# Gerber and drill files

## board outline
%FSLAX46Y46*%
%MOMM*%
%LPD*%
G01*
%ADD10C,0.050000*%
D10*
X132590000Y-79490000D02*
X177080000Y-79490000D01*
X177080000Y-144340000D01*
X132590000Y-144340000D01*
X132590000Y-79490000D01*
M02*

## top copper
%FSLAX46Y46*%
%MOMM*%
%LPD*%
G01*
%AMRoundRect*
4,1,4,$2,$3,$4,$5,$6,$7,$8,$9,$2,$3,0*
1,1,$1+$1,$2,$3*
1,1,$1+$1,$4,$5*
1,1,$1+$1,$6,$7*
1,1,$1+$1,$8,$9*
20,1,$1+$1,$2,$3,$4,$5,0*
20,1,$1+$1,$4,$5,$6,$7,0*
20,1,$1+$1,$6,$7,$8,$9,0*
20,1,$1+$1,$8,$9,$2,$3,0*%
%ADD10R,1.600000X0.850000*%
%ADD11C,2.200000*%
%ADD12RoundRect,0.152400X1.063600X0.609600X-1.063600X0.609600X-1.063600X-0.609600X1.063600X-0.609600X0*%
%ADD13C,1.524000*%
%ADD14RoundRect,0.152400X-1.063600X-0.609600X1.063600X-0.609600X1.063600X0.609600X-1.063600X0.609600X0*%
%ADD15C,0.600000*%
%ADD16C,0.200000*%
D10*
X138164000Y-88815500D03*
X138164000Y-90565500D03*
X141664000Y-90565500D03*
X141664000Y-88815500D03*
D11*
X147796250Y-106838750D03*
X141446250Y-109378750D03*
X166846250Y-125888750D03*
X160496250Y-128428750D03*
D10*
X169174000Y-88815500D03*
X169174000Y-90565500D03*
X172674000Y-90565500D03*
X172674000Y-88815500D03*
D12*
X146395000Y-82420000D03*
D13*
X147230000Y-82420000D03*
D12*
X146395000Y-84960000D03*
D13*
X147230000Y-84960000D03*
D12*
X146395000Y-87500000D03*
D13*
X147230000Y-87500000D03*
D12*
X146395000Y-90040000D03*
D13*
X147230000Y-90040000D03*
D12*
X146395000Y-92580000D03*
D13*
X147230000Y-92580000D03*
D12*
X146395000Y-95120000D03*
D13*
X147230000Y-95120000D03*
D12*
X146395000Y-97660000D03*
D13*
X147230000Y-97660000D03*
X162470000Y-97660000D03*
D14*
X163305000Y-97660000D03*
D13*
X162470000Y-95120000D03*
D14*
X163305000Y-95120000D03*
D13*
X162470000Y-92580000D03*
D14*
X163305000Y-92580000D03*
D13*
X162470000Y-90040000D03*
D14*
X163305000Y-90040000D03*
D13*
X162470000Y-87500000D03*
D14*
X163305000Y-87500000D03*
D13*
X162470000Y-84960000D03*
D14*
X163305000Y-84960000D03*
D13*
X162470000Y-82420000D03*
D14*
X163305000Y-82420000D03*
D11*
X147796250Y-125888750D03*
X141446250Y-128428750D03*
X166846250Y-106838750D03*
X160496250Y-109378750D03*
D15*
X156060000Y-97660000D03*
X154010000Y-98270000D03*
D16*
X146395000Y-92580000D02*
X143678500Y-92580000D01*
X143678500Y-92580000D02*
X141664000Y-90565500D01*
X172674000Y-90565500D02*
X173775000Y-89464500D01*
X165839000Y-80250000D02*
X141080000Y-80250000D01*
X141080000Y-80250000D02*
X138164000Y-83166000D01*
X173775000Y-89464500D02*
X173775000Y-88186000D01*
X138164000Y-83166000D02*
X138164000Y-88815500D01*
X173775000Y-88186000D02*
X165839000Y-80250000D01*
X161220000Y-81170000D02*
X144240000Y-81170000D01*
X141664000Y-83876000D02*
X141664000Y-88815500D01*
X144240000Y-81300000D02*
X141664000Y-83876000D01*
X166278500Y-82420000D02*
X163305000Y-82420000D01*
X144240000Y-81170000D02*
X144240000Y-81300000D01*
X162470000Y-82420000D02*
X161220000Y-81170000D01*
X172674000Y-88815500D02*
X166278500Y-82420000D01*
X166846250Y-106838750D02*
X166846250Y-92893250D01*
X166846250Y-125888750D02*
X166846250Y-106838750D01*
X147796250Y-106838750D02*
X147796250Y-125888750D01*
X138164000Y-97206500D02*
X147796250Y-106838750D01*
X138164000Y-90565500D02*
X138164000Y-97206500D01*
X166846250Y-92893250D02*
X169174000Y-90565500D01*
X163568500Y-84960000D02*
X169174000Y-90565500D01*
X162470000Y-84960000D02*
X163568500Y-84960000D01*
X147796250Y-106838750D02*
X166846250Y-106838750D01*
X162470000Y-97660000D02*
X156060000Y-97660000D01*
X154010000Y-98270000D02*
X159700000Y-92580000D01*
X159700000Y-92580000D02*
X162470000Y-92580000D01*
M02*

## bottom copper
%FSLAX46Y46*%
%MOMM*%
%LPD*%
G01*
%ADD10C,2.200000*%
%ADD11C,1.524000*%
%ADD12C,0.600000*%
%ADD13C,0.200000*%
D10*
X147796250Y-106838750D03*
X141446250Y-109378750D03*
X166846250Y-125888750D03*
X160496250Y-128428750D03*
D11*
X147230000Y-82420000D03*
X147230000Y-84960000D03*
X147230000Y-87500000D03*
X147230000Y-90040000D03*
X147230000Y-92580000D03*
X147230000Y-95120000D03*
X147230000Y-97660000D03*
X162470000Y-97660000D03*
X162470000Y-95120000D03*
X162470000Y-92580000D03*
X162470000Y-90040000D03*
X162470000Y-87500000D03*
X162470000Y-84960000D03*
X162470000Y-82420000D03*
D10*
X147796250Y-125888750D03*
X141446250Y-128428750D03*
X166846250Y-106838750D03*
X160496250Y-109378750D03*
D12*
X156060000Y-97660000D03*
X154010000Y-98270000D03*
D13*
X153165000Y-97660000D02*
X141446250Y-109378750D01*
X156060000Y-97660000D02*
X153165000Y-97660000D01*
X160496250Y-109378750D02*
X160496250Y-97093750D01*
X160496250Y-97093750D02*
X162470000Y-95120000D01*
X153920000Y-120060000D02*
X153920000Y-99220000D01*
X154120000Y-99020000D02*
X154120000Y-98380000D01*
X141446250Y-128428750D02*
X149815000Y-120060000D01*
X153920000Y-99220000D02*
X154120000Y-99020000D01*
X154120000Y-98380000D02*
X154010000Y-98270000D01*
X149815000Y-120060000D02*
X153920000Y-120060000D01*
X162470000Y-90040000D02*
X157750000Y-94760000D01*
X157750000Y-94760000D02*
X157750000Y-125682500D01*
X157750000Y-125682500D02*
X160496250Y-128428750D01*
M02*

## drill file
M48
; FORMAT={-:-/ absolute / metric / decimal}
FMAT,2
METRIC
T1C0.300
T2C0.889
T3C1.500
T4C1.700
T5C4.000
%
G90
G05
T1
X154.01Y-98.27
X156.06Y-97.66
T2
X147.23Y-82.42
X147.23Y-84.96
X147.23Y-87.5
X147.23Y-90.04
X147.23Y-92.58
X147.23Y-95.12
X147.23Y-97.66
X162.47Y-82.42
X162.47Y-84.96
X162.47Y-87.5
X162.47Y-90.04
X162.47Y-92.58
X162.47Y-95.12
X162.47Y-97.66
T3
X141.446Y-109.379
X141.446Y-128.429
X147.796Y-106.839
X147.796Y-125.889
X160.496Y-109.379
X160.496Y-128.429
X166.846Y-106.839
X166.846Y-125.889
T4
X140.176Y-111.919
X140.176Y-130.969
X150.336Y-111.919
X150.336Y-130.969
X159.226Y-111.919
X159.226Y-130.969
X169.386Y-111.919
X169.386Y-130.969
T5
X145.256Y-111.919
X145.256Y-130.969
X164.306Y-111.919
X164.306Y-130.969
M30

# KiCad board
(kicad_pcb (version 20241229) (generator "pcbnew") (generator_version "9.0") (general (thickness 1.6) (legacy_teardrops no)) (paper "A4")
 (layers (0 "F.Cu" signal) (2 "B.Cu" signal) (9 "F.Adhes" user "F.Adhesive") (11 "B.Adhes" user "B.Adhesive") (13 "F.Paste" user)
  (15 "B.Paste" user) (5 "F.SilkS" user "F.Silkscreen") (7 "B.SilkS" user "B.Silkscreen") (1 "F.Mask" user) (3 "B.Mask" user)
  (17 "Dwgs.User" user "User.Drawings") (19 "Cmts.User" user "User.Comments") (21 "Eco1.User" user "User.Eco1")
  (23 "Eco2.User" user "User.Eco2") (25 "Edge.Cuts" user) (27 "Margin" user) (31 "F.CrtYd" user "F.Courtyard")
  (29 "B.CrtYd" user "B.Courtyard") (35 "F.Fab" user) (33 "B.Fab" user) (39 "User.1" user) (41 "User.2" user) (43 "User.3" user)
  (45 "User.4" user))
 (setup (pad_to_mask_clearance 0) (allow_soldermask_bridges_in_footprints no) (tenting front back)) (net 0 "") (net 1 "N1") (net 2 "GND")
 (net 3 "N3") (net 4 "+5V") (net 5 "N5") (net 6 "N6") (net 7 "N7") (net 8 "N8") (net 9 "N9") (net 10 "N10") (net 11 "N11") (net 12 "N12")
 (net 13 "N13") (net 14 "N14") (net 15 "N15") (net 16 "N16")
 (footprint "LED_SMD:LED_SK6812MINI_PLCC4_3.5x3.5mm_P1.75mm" (layer "F.Cu") (at 139.914 89.6905)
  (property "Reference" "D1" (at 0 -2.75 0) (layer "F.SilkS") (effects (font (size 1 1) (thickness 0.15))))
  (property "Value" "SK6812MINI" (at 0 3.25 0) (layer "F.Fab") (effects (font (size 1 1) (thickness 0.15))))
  (pad "1" smd rect (at -1.75 -0.875) (size 1.6 0.85) (layers "F.Cu" "F.Mask" "F.Paste") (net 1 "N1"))
  (pad "2" smd rect (at -1.75 0.875) (size 1.6 0.85) (layers "F.Cu" "F.Mask" "F.Paste") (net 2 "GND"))
  (pad "3" smd rect (at 1.75 0.875) (size 1.6 0.85) (layers "F.Cu" "F.Mask" "F.Paste") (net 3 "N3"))
  (pad "4" smd rect (at 1.75 -0.875) (size 1.6 0.85) (layers "F.Cu" "F.Mask" "F.Paste") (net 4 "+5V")))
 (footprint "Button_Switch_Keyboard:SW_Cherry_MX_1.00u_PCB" (layer "F.Cu") (at 147.79625 106.83875)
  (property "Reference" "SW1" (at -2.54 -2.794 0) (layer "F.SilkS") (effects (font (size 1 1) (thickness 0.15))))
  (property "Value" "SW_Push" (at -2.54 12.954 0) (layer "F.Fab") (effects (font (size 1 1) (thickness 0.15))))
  (pad "" np_thru_hole circle (at -7.62 5.08) (size 1.7 1.7) (drill 1.7) (layers "*.Cu" "*.Mask"))
  (pad "" np_thru_hole circle (at -2.54 5.08) (size 4 4) (drill 4) (layers "*.Cu" "*.Mask"))
  (pad "" np_thru_hole circle (at 2.54 5.08) (size 1.7 1.7) (drill 1.7) (layers "*.Cu" "*.Mask"))
  (pad "1" thru_hole circle (at 0 0) (size 2.2 2.2) (drill 1.5) (layers "*.Cu" "*.Mask") (remove_unused_layers no) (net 2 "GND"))
  (pad "2" thru_hole circle (at -6.35 2.54) (size 2.2 2.2) (drill 1.5) (layers "*.Cu" "*.Mask") (remove_unused_layers no) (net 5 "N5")))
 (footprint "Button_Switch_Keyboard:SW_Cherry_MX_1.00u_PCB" (layer "F.Cu") (at 166.84625 125.88875)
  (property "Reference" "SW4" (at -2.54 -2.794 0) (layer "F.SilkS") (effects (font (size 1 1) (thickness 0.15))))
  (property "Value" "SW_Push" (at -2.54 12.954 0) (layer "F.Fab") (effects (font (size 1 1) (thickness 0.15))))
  (pad "" np_thru_hole circle (at -7.62 5.08) (size 1.7 1.7) (drill 1.7) (layers "*.Cu" "*.Mask"))
  (pad "" np_thru_hole circle (at -2.54 5.08) (size 4 4) (drill 4) (layers "*.Cu" "*.Mask"))
  (pad "" np_thru_hole circle (at 2.54 5.08) (size 1.7 1.7) (drill 1.7) (layers "*.Cu" "*.Mask"))
  (pad "1" thru_hole circle (at 0 0) (size 2.2 2.2) (drill 1.5) (layers "*.Cu" "*.Mask") (remove_unused_layers no) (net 2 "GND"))
  (pad "2" thru_hole circle (at -6.35 2.54) (size 2.2 2.2) (drill 1.5) (layers "*.Cu" "*.Mask") (remove_unused_layers no) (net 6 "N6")))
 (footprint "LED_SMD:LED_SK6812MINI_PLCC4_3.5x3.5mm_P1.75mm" (layer "F.Cu") (at 170.924 89.6905)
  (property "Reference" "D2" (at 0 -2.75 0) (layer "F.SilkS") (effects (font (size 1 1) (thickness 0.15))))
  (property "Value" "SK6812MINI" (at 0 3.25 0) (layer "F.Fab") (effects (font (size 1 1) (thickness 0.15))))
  (pad "1" smd rect (at -1.75 -0.875) (size 1.6 0.85) (layers "F.Cu" "F.Mask" "F.Paste") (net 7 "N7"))
  (pad "2" smd rect (at -1.75 0.875) (size 1.6 0.85) (layers "F.Cu" "F.Mask" "F.Paste") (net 2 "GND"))
  (pad "3" smd rect (at 1.75 0.875) (size 1.6 0.85) (layers "F.Cu" "F.Mask" "F.Paste") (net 1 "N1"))
  (pad "4" smd rect (at 1.75 -0.875) (size 1.6 0.85) (layers "F.Cu" "F.Mask" "F.Paste") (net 4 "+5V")))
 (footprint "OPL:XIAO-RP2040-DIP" (layer "F.Cu") (at 154.85 90.04)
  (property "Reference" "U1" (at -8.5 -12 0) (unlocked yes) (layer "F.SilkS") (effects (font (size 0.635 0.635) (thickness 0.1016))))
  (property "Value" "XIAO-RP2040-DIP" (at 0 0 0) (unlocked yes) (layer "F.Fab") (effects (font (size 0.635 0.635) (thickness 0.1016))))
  (pad "1" smd roundrect (at -8.455 -7.62 180) (size 2.432 1.524) (layers "F.Cu" "F.Mask") (roundrect_rratio 0.1) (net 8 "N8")
   (thermal_bridge_angle 45))
  (pad "1" thru_hole circle (at -7.62 -7.62 180) (size 1.524 1.524) (drill 0.889) (layers "*.Cu" "*.Mask") (remove_unused_layers no)
   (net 8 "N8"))
  (pad "2" smd roundrect (at -8.455 -5.08 180) (size 2.432 1.524) (layers "F.Cu" "F.Mask") (roundrect_rratio 0.1) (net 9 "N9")
   (thermal_bridge_angle 45))
  (pad "2" thru_hole circle (at -7.62 -5.08 180) (size 1.524 1.524) (drill 0.889) (layers "*.Cu" "*.Mask") (remove_unused_layers no)
   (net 9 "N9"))
  (pad "3" smd roundrect (at -8.455 -2.54 180) (size 2.432 1.524) (layers "F.Cu" "F.Mask") (roundrect_rratio 0.1) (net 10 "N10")
   (thermal_bridge_angle 45))
  (pad "3" thru_hole circle (at -7.62 -2.54 180) (size 1.524 1.524) (drill 0.889) (layers "*.Cu" "*.Mask") (remove_unused_layers no)
   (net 10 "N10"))
  (pad "4" smd roundrect (at -8.455 0 180) (size 2.432 1.524) (layers "F.Cu" "F.Mask") (roundrect_rratio 0.1) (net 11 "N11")
   (thermal_bridge_angle 45))
  (pad "4" thru_hole circle (at -7.62 0 180) (size 1.524 1.524) (drill 0.889) (layers "*.Cu" "*.Mask") (remove_unused_layers no)
   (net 11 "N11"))
  (pad "5" smd roundrect (at -8.455 2.54 180) (size 2.432 1.524) (layers "F.Cu" "F.Mask") (roundrect_rratio 0.1) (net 3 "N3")
   (thermal_bridge_angle 45))
  (pad "5" thru_hole circle (at -7.62 2.54 180) (size 1.524 1.524) (drill 0.889) (layers "*.Cu" "*.Mask") (remove_unused_layers no)
   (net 3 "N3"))
  (pad "6" smd roundrect (at -8.455 5.08 180) (size 2.432 1.524) (layers "F.Cu" "F.Mask") (roundrect_rratio 0.1) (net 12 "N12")
   (thermal_bridge_angle 45))
  (pad "6" thru_hole circle (at -7.62 5.08 180) (size 1.524 1.524) (drill 0.889) (layers "*.Cu" "*.Mask") (remove_unused_layers no)
   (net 12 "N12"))
  (pad "7" smd roundrect (at -8.455 7.62 180) (size 2.432 1.524) (layers "F.Cu" "F.Mask") (roundrect_rratio 0.1) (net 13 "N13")
   (thermal_bridge_angle 45))
  (pad "7" thru_hole circle (at -7.62 7.62 180) (size 1.524 1.524) (drill 0.889) (layers "*.Cu" "*.Mask") (remove_unused_layers no)
   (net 13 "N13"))
  (pad "8" thru_hole circle (at 7.62 7.62) (size 1.524 1.524) (drill 0.889) (layers "*.Cu" "*.Mask") (remove_unused_layers no) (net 5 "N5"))
  (pad "8" smd roundrect (at 8.455 7.62) (size 2.432 1.524) (layers "F.Cu" "F.Mask") (roundrect_rratio 0.1) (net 5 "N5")
   (thermal_bridge_angle 45))
  (pad "9" thru_hole circle (at 7.62 5.08) (size 1.524 1.524) (drill 0.889) (layers "*.Cu" "*.Mask") (remove_unused_layers no)
   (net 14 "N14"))
  (pad "9" smd roundrect (at 8.455 5.08) (size 2.432 1.524) (layers "F.Cu" "F.Mask") (roundrect_rratio 0.1) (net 14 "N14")
   (thermal_bridge_angle 45))
  (pad "10" thru_hole circle (at 7.62 2.54) (size 1.524 1.524) (drill 0.889) (layers "*.Cu" "*.Mask") (remove_unused_layers no)
   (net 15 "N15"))
  (pad "10" smd roundrect (at 8.455 2.54) (size 2.432 1.524) (layers "F.Cu" "F.Mask") (roundrect_rratio 0.1) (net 15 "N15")
   (thermal_bridge_angle 45))
  (pad "11" thru_hole circle (at 7.62 0) (size 1.524 1.524) (drill 0.889) (layers "*.Cu" "*.Mask") (remove_unused_layers no) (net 6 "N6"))
  (pad "11" smd roundrect (at 8.455 0) (size 2.432 1.524) (layers "F.Cu" "F.Mask") (roundrect_rratio 0.1) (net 6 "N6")
   (thermal_bridge_angle 45))
  (pad "12" thru_hole circle (at 7.62 -2.54) (size 1.524 1.524) (drill 0.889) (layers "*.Cu" "*.Mask") (remove_unused_layers no)
   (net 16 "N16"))
  (pad "12" smd roundrect (at 8.455 -2.54) (size 2.432 1.524) (layers "F.Cu" "F.Mask") (roundrect_rratio 0.1) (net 16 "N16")
   (thermal_bridge_angle 45))
  (pad "13" thru_hole circle (at 7.62 -5.08) (size 1.524 1.524) (drill 0.889) (layers "*.Cu" "*.Mask") (remove_unused_layers no)
   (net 2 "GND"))
  (pad "13" smd roundrect (at 8.455 -5.08) (size 2.432 1.524) (layers "F.Cu" "F.Mask") (roundrect_rratio 0.1) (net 2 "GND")
   (thermal_bridge_angle 45))
  (pad "14" thru_hole circle (at 7.62 -7.62) (size 1.524 1.524) (drill 0.889) (layers "*.Cu" "*.Mask") (remove_unused_layers no)
   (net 4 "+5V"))
  (pad "14" smd roundrect (at 8.455 -7.62) (size 2.432 1.524) (layers "F.Cu" "F.Mask") (roundrect_rratio 0.1) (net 4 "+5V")
   (thermal_bridge_angle 45)))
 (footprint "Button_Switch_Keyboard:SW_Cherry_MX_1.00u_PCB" (layer "F.Cu") (at 147.79625 125.88875)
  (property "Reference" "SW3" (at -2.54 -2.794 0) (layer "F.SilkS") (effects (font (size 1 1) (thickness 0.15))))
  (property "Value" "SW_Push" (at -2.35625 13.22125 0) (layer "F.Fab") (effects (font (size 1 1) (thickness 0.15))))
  (pad "" np_thru_hole circle (at -7.62 5.08) (size 1.7 1.7) (drill 1.7) (layers "*.Cu" "*.Mask"))
  (pad "" np_thru_hole circle (at -2.54 5.08) (size 4 4) (drill 4) (layers "*.Cu" "*.Mask"))
  (pad "" np_thru_hole circle (at 2.54 5.08) (size 1.7 1.7) (drill 1.7) (layers "*.Cu" "*.Mask"))
  (pad "1" thru_hole circle (at 0 0) (size 2.2 2.2) (drill 1.5) (layers "*.Cu" "*.Mask") (remove_unused_layers no) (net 2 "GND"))
  (pad "2" thru_hole circle (at -6.35 2.54) (size 2.2 2.2) (drill 1.5) (layers "*.Cu" "*.Mask") (remove_unused_layers no) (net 15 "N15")))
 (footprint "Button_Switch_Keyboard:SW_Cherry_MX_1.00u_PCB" (layer "F.Cu") (at 166.84625 106.83875)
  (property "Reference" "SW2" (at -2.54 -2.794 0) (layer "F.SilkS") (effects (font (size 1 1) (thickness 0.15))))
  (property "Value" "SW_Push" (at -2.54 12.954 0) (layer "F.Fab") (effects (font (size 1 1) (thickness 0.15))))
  (pad "" np_thru_hole circle (at -7.62 5.08) (size 1.7 1.7) (drill 1.7) (layers "*.Cu" "*.Mask"))
  (pad "" np_thru_hole circle (at -2.54 5.08) (size 4 4) (drill 4) (layers "*.Cu" "*.Mask"))
  (pad "" np_thru_hole circle (at 2.54 5.08) (size 1.7 1.7) (drill 1.7) (layers "*.Cu" "*.Mask"))
  (pad "1" thru_hole circle (at 0 0) (size 2.2 2.2) (drill 1.5) (layers "*.Cu" "*.Mask") (remove_unused_layers no) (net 2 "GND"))
  (pad "2" thru_hole circle (at -6.35 2.54) (size 2.2 2.2) (drill 1.5) (layers "*.Cu" "*.Mask") (remove_unused_layers no) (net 14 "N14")))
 (gr_rect (start 132.59 79.49) (end 177.08 144.34) (stroke (width 0.05) (type default)) (fill no) (layer "Edge.Cuts"))
 (segment (start 146.395 92.58) (end 143.6785 92.58) (width 0.2) (layer "F.Cu") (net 3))
 (segment (start 143.6785 92.58) (end 141.664 90.5655) (width 0.2) (layer "F.Cu") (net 3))
 (segment (start 172.674 90.5655) (end 173.775 89.4645) (width 0.2) (layer "F.Cu") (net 1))
 (segment (start 165.839 80.25) (end 141.08 80.25) (width 0.2) (layer "F.Cu") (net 1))
 (segment (start 141.08 80.25) (end 138.164 83.166) (width 0.2) (layer "F.Cu") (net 1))
 (segment (start 173.775 89.4645) (end 173.775 88.186) (width 0.2) (layer "F.Cu") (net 1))
 (segment (start 138.164 83.166) (end 138.164 88.8155) (width 0.2) (layer "F.Cu") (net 1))
 (segment (start 173.775 88.186) (end 165.839 80.25) (width 0.2) (layer "F.Cu") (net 1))
 (segment (start 161.22 81.17) (end 144.24 81.17) (width 0.2) (layer "F.Cu") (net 4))
 (segment (start 141.664 83.876) (end 141.664 88.8155) (width 0.2) (layer "F.Cu") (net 4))
 (segment (start 144.24 81.3) (end 141.664 83.876) (width 0.2) (layer "F.Cu") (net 4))
 (segment (start 166.2785 82.42) (end 163.305 82.42) (width 0.2) (layer "F.Cu") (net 4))
 (segment (start 144.24 81.17) (end 144.24 81.3) (width 0.2) (layer "F.Cu") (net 4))
 (segment (start 162.47 82.42) (end 161.22 81.17) (width 0.2) (layer "F.Cu") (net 4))
 (segment (start 172.674 88.8155) (end 166.2785 82.42) (width 0.2) (layer "F.Cu") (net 4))
 (segment (start 166.84625 106.83875) (end 166.84625 92.89325) (width 0.2) (layer "F.Cu") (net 2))
 (segment (start 166.84625 125.88875) (end 166.84625 106.83875) (width 0.2) (layer "F.Cu") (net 2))
 (segment (start 147.79625 106.83875) (end 147.79625 125.88875) (width 0.2) (layer "F.Cu") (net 2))
 (segment (start 138.164 97.2065) (end 147.79625 106.83875) (width 0.2) (layer "F.Cu") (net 2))
 (segment (start 138.164 90.5655) (end 138.164 97.2065) (width 0.2) (layer "F.Cu") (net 2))
 (segment (start 166.84625 92.89325) (end 169.174 90.5655) (width 0.2) (layer "F.Cu") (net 2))
 (segment (start 163.5685 84.96) (end 169.174 90.5655) (width 0.2) (layer "F.Cu") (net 2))
 (segment (start 162.47 84.96) (end 163.5685 84.96) (width 0.2) (layer "F.Cu") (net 2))
 (segment (start 147.79625 106.83875) (end 166.84625 106.83875) (width 0.2) (layer "F.Cu") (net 2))
 (segment (start 162.47 97.66) (end 156.06 97.66) (width 0.2) (layer "F.Cu") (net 5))
 (via (at 156.06 97.66) (size 0.6) (drill 0.3) (layers "F.Cu" "B.Cu") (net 5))
 (segment (start 153.165 97.66) (end 141.44625 109.37875) (width 0.2) (layer "B.Cu") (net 5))
 (segment (start 156.06 97.66) (end 153.165 97.66) (width 0.2) (layer "B.Cu") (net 5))
 (segment (start 160.49625 109.37875) (end 160.49625 97.09375) (width 0.2) (layer "B.Cu") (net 14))
 (segment (start 160.49625 97.09375) (end 162.47 95.12) (width 0.2) (layer "B.Cu") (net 14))
 (segment (start 154.01 98.27) (end 159.7 92.58) (width 0.2) (layer "F.Cu") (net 15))
 (segment (start 159.7 92.58) (end 162.47 92.58) (width 0.2) (layer "F.Cu") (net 15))
 (via (at 154.01 98.27) (size 0.6) (drill 0.3) (layers "F.Cu" "B.Cu") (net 15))
 (segment (start 153.92 120.06) (end 153.92 99.22) (width 0.2) (layer "B.Cu") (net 15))
 (segment (start 154.12 99.02) (end 154.12 98.38) (width 0.2) (layer "B.Cu") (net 15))
 (segment (start 141.44625 128.42875) (end 149.815 120.06) (width 0.2) (layer "B.Cu") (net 15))
 (segment (start 153.92 99.22) (end 154.12 99.02) (width 0.2) (layer "B.Cu") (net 15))
 (segment (start 154.12 98.38) (end 154.01 98.27) (width 0.2) (layer "B.Cu") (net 15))
 (segment (start 149.815 120.06) (end 153.92 120.06) (width 0.2) (layer "B.Cu") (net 15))
 (segment (start 162.47 90.04) (end 157.75 94.76) (width 0.2) (layer "B.Cu") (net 6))
 (segment (start 157.75 94.76) (end 157.75 125.6825) (width 0.2) (layer "B.Cu") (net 6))
 (segment (start 157.75 125.6825) (end 160.49625 128.42875) (width 0.2) (layer "B.Cu") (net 6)))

